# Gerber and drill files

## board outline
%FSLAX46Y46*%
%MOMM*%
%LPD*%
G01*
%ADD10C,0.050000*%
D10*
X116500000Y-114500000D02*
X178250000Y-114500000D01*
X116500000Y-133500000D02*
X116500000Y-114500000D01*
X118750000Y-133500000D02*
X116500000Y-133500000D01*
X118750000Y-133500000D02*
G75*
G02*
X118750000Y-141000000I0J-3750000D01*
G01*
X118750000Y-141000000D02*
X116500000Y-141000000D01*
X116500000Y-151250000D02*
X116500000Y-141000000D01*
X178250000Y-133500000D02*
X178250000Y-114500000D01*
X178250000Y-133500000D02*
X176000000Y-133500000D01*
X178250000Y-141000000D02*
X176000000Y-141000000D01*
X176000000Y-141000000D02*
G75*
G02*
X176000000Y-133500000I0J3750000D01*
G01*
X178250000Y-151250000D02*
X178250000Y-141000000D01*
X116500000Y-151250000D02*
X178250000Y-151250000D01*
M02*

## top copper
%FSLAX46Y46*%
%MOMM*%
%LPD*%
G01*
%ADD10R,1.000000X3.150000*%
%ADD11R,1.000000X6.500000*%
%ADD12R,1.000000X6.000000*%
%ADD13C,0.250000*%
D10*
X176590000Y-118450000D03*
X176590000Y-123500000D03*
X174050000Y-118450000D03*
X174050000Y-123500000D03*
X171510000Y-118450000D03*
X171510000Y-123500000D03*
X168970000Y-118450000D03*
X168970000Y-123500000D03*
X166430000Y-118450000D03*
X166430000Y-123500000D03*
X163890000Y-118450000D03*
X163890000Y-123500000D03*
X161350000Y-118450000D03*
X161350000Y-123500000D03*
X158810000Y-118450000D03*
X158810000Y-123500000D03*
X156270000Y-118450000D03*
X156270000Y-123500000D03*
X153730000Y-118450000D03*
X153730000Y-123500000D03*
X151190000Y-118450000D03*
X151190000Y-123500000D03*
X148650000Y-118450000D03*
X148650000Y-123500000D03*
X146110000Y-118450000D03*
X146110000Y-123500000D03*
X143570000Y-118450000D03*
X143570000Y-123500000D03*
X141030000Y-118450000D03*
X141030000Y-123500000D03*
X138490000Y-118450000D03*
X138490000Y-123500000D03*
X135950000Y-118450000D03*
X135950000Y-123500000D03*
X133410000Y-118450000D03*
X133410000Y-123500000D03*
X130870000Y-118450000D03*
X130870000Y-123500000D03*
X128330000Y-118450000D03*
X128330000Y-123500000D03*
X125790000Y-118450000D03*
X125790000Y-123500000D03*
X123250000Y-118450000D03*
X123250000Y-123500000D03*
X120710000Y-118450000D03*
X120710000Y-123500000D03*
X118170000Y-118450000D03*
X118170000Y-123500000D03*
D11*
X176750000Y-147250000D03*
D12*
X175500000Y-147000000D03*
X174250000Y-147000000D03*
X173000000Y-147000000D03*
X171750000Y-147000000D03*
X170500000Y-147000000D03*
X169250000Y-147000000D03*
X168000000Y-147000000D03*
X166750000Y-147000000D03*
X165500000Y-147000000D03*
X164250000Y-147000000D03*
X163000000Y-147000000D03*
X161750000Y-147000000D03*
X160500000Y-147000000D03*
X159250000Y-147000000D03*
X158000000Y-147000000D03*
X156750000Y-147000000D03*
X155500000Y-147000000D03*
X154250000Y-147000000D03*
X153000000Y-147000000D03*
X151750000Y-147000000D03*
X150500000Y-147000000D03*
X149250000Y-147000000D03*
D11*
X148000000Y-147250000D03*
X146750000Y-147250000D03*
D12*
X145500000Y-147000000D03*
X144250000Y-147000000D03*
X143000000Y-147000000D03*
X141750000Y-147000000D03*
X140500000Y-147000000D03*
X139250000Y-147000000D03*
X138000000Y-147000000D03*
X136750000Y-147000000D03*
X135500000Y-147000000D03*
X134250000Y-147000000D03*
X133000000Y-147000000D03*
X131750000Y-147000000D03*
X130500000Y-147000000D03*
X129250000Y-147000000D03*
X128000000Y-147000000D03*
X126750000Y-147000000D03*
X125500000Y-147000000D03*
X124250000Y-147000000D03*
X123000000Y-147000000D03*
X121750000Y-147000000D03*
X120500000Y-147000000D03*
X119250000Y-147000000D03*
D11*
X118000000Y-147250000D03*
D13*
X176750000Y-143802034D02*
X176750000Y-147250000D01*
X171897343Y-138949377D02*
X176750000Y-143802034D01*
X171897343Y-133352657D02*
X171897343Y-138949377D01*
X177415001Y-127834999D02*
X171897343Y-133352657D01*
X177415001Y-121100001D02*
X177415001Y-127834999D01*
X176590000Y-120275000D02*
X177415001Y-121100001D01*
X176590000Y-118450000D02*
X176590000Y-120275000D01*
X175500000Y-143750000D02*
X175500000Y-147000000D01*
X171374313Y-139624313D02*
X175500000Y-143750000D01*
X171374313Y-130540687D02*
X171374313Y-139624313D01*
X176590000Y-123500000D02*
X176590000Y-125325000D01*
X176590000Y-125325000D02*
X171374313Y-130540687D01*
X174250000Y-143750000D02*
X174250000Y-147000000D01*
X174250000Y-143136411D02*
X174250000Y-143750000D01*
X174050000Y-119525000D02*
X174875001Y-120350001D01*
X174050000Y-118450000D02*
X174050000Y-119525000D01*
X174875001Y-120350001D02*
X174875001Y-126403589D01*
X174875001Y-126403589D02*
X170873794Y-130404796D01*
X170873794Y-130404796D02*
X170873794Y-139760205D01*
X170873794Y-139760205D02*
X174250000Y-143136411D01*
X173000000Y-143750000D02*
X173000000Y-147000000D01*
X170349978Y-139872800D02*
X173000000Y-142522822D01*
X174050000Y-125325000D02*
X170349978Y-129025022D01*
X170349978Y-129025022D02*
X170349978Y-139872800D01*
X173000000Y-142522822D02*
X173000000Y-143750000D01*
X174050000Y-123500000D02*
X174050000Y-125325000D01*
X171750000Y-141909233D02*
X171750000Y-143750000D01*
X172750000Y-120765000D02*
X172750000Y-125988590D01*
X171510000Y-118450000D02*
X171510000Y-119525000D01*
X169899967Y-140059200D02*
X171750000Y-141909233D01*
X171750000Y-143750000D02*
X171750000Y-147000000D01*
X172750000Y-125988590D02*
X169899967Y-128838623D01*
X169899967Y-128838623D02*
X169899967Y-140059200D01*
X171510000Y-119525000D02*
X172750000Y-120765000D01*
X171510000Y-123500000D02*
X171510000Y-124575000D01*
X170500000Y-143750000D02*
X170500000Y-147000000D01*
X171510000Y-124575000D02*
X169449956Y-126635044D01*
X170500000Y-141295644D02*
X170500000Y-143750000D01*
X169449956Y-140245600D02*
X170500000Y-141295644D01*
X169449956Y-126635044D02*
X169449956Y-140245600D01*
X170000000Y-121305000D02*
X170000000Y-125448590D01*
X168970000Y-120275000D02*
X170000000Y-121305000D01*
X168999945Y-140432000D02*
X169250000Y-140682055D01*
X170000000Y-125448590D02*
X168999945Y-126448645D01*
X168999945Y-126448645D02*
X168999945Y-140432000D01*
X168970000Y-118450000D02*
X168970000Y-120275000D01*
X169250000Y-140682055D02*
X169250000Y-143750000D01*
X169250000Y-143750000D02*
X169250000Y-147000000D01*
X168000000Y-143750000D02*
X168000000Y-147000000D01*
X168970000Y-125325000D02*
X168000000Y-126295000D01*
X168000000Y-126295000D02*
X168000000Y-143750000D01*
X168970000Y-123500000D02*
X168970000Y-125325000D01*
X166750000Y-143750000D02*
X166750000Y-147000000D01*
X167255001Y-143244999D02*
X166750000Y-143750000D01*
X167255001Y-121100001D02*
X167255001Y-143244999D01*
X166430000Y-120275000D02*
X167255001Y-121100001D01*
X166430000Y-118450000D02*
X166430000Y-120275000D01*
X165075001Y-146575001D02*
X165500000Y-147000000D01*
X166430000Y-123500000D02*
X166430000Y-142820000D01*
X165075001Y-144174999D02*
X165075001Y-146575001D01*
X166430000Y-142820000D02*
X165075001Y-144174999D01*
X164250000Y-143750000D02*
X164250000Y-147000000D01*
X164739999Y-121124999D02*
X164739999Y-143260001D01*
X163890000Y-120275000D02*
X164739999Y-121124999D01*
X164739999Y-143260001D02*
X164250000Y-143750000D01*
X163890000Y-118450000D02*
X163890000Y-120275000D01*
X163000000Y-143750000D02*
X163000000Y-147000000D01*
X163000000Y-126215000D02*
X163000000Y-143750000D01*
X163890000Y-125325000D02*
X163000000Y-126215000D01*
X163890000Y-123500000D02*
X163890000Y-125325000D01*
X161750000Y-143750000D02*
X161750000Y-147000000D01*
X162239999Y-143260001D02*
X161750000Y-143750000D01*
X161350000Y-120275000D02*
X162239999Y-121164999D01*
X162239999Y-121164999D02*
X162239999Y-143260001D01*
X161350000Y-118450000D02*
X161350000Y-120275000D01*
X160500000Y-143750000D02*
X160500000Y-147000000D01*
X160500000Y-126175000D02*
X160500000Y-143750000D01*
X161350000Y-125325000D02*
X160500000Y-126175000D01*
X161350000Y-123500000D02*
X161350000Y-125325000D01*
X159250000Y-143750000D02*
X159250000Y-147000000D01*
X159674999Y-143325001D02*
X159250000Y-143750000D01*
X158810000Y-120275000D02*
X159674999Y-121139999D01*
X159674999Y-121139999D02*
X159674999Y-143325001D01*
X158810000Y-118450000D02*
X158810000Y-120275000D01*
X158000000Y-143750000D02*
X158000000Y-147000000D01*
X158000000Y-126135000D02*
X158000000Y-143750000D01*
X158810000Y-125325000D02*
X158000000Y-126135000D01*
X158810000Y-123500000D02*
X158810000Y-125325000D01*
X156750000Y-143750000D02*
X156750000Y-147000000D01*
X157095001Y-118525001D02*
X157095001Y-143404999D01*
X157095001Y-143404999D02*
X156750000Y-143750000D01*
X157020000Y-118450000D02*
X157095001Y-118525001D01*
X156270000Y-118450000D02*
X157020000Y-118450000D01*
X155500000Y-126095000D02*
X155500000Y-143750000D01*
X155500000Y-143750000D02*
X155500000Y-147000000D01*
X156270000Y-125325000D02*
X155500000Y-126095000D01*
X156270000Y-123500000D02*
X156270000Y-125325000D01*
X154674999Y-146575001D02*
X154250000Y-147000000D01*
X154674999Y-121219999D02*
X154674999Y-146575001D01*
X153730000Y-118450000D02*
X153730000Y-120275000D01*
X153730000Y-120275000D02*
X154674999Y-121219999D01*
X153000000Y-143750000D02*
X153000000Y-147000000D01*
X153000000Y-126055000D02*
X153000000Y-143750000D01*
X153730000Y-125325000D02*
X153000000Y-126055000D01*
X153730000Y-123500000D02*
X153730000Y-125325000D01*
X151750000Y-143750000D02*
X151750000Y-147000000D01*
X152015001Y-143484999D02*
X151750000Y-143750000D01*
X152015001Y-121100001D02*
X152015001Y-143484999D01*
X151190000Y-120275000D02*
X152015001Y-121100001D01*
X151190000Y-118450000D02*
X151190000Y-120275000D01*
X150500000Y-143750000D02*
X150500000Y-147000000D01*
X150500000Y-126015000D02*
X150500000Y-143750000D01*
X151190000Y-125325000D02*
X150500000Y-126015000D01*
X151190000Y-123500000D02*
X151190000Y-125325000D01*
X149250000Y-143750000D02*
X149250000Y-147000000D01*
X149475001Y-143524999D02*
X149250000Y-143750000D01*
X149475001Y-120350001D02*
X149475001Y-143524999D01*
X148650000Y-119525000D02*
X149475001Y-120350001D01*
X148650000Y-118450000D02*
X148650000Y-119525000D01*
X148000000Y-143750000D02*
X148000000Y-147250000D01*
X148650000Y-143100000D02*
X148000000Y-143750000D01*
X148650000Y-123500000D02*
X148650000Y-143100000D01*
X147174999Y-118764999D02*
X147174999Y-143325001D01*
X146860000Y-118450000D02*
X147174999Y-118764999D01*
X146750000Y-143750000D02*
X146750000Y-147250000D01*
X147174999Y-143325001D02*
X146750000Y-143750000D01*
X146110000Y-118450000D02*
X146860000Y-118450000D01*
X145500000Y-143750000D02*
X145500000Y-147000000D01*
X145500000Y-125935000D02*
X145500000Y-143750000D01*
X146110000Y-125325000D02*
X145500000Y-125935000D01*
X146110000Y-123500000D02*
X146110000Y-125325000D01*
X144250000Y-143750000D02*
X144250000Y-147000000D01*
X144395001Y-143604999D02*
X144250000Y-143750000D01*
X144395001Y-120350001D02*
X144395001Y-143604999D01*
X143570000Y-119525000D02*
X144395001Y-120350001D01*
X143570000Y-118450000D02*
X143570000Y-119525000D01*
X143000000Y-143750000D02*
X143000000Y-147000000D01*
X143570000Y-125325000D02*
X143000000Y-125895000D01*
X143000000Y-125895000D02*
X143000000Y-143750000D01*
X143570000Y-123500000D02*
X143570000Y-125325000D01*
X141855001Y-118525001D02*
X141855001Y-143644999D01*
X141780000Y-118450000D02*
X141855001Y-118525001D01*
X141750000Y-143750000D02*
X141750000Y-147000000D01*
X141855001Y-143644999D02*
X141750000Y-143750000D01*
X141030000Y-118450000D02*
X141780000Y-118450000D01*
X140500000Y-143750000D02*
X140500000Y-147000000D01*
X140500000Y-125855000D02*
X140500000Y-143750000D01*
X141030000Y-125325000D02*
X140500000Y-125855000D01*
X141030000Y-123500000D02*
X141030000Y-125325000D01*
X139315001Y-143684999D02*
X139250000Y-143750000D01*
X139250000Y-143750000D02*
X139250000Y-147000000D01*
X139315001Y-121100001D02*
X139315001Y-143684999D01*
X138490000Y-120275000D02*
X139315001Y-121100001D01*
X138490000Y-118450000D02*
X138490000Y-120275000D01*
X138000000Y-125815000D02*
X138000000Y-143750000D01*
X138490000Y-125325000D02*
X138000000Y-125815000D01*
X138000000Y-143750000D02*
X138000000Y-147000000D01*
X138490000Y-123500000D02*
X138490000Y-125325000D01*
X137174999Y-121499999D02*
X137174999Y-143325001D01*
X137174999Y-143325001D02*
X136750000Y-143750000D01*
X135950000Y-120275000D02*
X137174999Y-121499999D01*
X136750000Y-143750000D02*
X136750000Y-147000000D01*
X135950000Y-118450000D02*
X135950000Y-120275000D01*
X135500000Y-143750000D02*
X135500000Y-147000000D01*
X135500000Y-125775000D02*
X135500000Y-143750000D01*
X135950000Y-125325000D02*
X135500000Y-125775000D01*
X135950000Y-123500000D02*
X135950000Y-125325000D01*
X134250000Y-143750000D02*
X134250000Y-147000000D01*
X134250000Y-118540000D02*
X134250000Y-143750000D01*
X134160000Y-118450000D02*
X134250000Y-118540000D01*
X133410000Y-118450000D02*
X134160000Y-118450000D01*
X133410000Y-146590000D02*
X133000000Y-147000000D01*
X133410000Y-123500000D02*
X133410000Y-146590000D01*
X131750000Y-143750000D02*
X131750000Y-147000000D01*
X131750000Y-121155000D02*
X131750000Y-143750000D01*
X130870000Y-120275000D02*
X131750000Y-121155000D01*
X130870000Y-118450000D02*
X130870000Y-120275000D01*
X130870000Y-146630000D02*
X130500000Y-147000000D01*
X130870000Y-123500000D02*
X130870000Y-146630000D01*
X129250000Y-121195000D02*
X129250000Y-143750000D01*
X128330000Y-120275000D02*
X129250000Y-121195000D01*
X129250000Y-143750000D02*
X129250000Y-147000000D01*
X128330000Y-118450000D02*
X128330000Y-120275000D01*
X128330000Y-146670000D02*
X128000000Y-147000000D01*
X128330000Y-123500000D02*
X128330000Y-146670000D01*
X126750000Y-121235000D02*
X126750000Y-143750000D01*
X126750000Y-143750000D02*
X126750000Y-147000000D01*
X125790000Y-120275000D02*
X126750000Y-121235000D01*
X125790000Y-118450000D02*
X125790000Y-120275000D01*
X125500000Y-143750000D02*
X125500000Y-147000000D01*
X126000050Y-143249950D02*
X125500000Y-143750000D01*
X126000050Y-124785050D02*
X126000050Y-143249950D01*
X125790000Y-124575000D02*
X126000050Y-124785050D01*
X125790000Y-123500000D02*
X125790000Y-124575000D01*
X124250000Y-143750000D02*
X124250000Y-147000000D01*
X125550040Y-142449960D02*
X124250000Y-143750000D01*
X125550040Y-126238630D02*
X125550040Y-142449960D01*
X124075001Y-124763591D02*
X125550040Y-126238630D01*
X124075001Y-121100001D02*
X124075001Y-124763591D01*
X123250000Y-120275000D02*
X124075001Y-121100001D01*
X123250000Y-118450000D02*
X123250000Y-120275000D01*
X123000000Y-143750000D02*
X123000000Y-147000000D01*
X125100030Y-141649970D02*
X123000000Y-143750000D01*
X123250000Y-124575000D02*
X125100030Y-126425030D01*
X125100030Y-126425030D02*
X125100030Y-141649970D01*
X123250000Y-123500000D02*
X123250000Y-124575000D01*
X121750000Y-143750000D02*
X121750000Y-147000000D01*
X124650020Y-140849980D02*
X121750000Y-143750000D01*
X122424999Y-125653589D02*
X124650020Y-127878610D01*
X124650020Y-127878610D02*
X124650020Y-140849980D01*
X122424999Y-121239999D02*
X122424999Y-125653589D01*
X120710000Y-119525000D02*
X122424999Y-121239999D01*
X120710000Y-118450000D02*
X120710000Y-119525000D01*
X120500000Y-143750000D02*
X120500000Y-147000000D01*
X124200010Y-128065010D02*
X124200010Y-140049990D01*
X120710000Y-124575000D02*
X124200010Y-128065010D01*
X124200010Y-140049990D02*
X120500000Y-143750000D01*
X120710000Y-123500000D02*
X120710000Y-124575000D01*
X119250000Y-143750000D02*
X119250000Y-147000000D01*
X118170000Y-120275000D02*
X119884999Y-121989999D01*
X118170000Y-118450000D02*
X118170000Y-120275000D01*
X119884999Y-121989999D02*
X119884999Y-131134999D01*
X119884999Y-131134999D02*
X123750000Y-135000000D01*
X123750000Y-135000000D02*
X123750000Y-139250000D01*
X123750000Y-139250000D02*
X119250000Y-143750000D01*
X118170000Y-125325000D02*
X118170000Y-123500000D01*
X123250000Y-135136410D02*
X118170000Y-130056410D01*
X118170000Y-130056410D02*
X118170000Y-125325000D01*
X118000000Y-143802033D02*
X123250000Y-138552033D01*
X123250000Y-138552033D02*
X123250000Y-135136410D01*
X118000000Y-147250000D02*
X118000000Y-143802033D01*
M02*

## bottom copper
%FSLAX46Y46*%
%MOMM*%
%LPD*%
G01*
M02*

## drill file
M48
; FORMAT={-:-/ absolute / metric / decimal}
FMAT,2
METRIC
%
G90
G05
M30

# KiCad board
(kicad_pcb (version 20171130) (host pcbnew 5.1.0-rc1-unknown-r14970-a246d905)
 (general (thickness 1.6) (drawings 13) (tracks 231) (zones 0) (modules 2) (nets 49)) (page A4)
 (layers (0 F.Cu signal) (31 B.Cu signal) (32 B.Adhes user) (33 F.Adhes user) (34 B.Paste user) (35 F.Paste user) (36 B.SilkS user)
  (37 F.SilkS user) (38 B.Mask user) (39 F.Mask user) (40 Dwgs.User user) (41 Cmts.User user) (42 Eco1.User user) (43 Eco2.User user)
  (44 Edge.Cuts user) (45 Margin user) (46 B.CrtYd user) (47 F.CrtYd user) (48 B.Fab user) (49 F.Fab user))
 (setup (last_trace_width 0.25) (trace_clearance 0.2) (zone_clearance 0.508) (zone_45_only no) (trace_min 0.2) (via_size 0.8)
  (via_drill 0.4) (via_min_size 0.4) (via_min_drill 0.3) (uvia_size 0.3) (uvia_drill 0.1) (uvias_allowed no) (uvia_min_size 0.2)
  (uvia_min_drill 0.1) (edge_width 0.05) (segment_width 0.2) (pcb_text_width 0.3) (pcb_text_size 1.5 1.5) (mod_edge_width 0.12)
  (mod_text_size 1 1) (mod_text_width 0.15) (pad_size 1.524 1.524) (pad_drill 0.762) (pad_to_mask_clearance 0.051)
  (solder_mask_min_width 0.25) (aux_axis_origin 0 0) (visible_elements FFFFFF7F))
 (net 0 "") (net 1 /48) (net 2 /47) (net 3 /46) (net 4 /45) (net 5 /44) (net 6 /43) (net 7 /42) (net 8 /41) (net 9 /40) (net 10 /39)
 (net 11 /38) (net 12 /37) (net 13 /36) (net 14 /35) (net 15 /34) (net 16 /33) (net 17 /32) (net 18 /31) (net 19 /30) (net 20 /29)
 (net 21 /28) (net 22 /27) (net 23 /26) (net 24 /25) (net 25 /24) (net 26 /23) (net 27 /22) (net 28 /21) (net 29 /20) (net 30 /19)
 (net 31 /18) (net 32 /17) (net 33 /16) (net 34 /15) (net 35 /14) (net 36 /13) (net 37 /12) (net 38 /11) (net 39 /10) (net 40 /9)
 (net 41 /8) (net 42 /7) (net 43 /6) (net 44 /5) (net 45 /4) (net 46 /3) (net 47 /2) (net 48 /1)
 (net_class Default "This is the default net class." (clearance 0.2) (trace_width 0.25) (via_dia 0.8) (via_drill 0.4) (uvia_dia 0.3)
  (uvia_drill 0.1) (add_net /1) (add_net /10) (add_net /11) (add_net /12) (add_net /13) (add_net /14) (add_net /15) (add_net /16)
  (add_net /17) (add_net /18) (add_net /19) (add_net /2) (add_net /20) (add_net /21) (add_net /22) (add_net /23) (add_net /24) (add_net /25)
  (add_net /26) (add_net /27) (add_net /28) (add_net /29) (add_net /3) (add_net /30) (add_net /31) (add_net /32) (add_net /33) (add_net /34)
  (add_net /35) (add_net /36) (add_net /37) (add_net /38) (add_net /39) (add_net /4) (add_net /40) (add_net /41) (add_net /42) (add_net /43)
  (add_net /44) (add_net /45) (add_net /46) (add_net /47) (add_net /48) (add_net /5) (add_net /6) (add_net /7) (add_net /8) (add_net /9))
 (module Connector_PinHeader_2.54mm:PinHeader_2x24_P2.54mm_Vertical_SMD (layer F.Cu) (at 147.38 120.975 90)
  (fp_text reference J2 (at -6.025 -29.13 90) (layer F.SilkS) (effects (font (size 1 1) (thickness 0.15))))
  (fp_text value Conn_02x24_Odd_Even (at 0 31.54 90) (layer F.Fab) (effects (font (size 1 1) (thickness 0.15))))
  (pad 48 smd rect (at 2.525 29.21 90) (size 3.15 1) (layers F.Cu F.Paste F.Mask) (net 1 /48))
  (pad 47 smd rect (at -2.525 29.21 90) (size 3.15 1) (layers F.Cu F.Paste F.Mask) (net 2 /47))
  (pad 46 smd rect (at 2.525 26.67 90) (size 3.15 1) (layers F.Cu F.Paste F.Mask) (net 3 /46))
  (pad 45 smd rect (at -2.525 26.67 90) (size 3.15 1) (layers F.Cu F.Paste F.Mask) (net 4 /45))
  (pad 44 smd rect (at 2.525 24.13 90) (size 3.15 1) (layers F.Cu F.Paste F.Mask) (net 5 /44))
  (pad 43 smd rect (at -2.525 24.13 90) (size 3.15 1) (layers F.Cu F.Paste F.Mask) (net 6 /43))
  (pad 42 smd rect (at 2.525 21.59 90) (size 3.15 1) (layers F.Cu F.Paste F.Mask) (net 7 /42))
  (pad 41 smd rect (at -2.525 21.59 90) (size 3.15 1) (layers F.Cu F.Paste F.Mask) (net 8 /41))
  (pad 40 smd rect (at 2.525 19.05 90) (size 3.15 1) (layers F.Cu F.Paste F.Mask) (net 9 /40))
  (pad 39 smd rect (at -2.525 19.05 90) (size 3.15 1) (layers F.Cu F.Paste F.Mask) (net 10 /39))
  (pad 38 smd rect (at 2.525 16.51 90) (size 3.15 1) (layers F.Cu F.Paste F.Mask) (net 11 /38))
  (pad 37 smd rect (at -2.525 16.51 90) (size 3.15 1) (layers F.Cu F.Paste F.Mask) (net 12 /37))
  (pad 36 smd rect (at 2.525 13.97 90) (size 3.15 1) (layers F.Cu F.Paste F.Mask) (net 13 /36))
  (pad 35 smd rect (at -2.525 13.97 90) (size 3.15 1) (layers F.Cu F.Paste F.Mask) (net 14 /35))
  (pad 34 smd rect (at 2.525 11.43 90) (size 3.15 1) (layers F.Cu F.Paste F.Mask) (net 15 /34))
  (pad 33 smd rect (at -2.525 11.43 90) (size 3.15 1) (layers F.Cu F.Paste F.Mask) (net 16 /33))
  (pad 32 smd rect (at 2.525 8.89 90) (size 3.15 1) (layers F.Cu F.Paste F.Mask) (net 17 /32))
  (pad 31 smd rect (at -2.525 8.89 90) (size 3.15 1) (layers F.Cu F.Paste F.Mask) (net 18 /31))
  (pad 30 smd rect (at 2.525 6.35 90) (size 3.15 1) (layers F.Cu F.Paste F.Mask) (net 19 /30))
  (pad 29 smd rect (at -2.525 6.35 90) (size 3.15 1) (layers F.Cu F.Paste F.Mask) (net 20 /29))
  (pad 28 smd rect (at 2.525 3.81 90) (size 3.15 1) (layers F.Cu F.Paste F.Mask) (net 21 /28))
  (pad 27 smd rect (at -2.525 3.81 90) (size 3.15 1) (layers F.Cu F.Paste F.Mask) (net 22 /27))
  (pad 26 smd rect (at 2.525 1.27 90) (size 3.15 1) (layers F.Cu F.Paste F.Mask) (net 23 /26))
  (pad 25 smd rect (at -2.525 1.27 90) (size 3.15 1) (layers F.Cu F.Paste F.Mask) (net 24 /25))
  (pad 24 smd rect (at 2.525 -1.27 90) (size 3.15 1) (layers F.Cu F.Paste F.Mask) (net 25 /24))
  (pad 23 smd rect (at -2.525 -1.27 90) (size 3.15 1) (layers F.Cu F.Paste F.Mask) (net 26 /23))
  (pad 22 smd rect (at 2.525 -3.81 90) (size 3.15 1) (layers F.Cu F.Paste F.Mask) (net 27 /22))
  (pad 21 smd rect (at -2.525 -3.81 90) (size 3.15 1) (layers F.Cu F.Paste F.Mask) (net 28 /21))
  (pad 20 smd rect (at 2.525 -6.35 90) (size 3.15 1) (layers F.Cu F.Paste F.Mask) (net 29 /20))
  (pad 19 smd rect (at -2.525 -6.35 90) (size 3.15 1) (layers F.Cu F.Paste F.Mask) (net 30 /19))
  (pad 18 smd rect (at 2.525 -8.89 90) (size 3.15 1) (layers F.Cu F.Paste F.Mask) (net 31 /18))
  (pad 17 smd rect (at -2.525 -8.89 90) (size 3.15 1) (layers F.Cu F.Paste F.Mask) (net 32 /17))
  (pad 16 smd rect (at 2.525 -11.43 90) (size 3.15 1) (layers F.Cu F.Paste F.Mask) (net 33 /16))
  (pad 15 smd rect (at -2.525 -11.43 90) (size 3.15 1) (layers F.Cu F.Paste F.Mask) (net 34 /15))
  (pad 14 smd rect (at 2.525 -13.97 90) (size 3.15 1) (layers F.Cu F.Paste F.Mask) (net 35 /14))
  (pad 13 smd rect (at -2.525 -13.97 90) (size 3.15 1) (layers F.Cu F.Paste F.Mask) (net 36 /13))
  (pad 12 smd rect (at 2.525 -16.51 90) (size 3.15 1) (layers F.Cu F.Paste F.Mask) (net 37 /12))
  (pad 11 smd rect (at -2.525 -16.51 90) (size 3.15 1) (layers F.Cu F.Paste F.Mask) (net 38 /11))
  (pad 10 smd rect (at 2.525 -19.05 90) (size 3.15 1) (layers F.Cu F.Paste F.Mask) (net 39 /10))
  (pad 9 smd rect (at -2.525 -19.05 90) (size 3.15 1) (layers F.Cu F.Paste F.Mask) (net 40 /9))
  (pad 8 smd rect (at 2.525 -21.59 90) (size 3.15 1) (layers F.Cu F.Paste F.Mask) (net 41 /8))
  (pad 7 smd rect (at -2.525 -21.59 90) (size 3.15 1) (layers F.Cu F.Paste F.Mask) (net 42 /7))
  (pad 6 smd rect (at 2.525 -24.13 90) (size 3.15 1) (layers F.Cu F.Paste F.Mask) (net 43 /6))
  (pad 5 smd rect (at -2.525 -24.13 90) (size 3.15 1) (layers F.Cu F.Paste F.Mask) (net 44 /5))
  (pad 4 smd rect (at 2.525 -26.67 90) (size 3.15 1) (layers F.Cu F.Paste F.Mask) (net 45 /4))
  (pad 3 smd rect (at -2.525 -26.67 90) (size 3.15 1) (layers F.Cu F.Paste F.Mask) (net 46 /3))
  (pad 2 smd rect (at 2.525 -29.21 90) (size 3.15 1) (layers F.Cu F.Paste F.Mask) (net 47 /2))
  (pad 1 smd rect (at -2.525 -29.21 90) (size 3.15 1) (layers F.Cu F.Paste F.Mask) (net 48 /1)))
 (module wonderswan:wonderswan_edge (layer F.Cu) (at 147.375 147)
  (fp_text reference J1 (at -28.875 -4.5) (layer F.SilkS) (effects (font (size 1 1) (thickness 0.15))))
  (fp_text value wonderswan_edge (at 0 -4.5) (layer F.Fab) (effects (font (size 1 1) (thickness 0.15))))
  (pad 48 smd rect (at 29.375 0.25) (size 1 6.5) (layers F.Cu F.Paste F.Mask) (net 1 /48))
  (pad 47 smd rect (at 28.125 0) (size 1 6) (layers F.Cu F.Paste F.Mask) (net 2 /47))
  (pad 46 smd rect (at 26.875 0) (size 1 6) (layers F.Cu F.Paste F.Mask) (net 3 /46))
  (pad 45 smd rect (at 25.625 0) (size 1 6) (layers F.Cu F.Paste F.Mask) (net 4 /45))
  (pad 44 smd rect (at 24.375 0) (size 1 6) (layers F.Cu F.Paste F.Mask) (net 5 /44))
  (pad 43 smd rect (at 23.125 0) (size 1 6) (layers F.Cu F.Paste F.Mask) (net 6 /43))
  (pad 42 smd rect (at 21.875 0) (size 1 6) (layers F.Cu F.Paste F.Mask) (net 7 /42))
  (pad 41 smd rect (at 20.625 0) (size 1 6) (layers F.Cu F.Paste F.Mask) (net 8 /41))
  (pad 40 smd rect (at 19.375 0) (size 1 6) (layers F.Cu F.Paste F.Mask) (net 9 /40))
  (pad 39 smd rect (at 18.125 0) (size 1 6) (layers F.Cu F.Paste F.Mask) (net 10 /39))
  (pad 38 smd rect (at 16.875 0) (size 1 6) (layers F.Cu F.Paste F.Mask) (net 11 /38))
  (pad 37 smd rect (at 15.625 0) (size 1 6) (layers F.Cu F.Paste F.Mask) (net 12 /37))
  (pad 36 smd rect (at 14.375 0) (size 1 6) (layers F.Cu F.Paste F.Mask) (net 13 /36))
  (pad 35 smd rect (at 13.125 0) (size 1 6) (layers F.Cu F.Paste F.Mask) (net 14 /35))
  (pad 34 smd rect (at 11.875 0) (size 1 6) (layers F.Cu F.Paste F.Mask) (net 15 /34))
  (pad 33 smd rect (at 10.625 0) (size 1 6) (layers F.Cu F.Paste F.Mask) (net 16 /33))
  (pad 32 smd rect (at 9.375 0) (size 1 6) (layers F.Cu F.Paste F.Mask) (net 17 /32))
  (pad 31 smd rect (at 8.125 0) (size 1 6) (layers F.Cu F.Paste F.Mask) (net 18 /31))
  (pad 30 smd rect (at 6.875 0) (size 1 6) (layers F.Cu F.Paste F.Mask) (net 19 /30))
  (pad 29 smd rect (at 5.625 0) (size 1 6) (layers F.Cu F.Paste F.Mask) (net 20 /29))
  (pad 28 smd rect (at 4.375 0) (size 1 6) (layers F.Cu F.Paste F.Mask) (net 21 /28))
  (pad 27 smd rect (at 3.125 0) (size 1 6) (layers F.Cu F.Paste F.Mask) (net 22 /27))
  (pad 26 smd rect (at 1.875 0) (size 1 6) (layers F.Cu F.Paste F.Mask) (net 23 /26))
  (pad 25 smd rect (at 0.625 0.25) (size 1 6.5) (layers F.Cu F.Paste F.Mask) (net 24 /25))
  (pad 24 smd rect (at -0.625 0.25) (size 1 6.5) (layers F.Cu F.Paste F.Mask) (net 25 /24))
  (pad 23 smd rect (at -1.875 0) (size 1 6) (layers F.Cu F.Paste F.Mask) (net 26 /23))
  (pad 22 smd rect (at -3.125 0) (size 1 6) (layers F.Cu F.Paste F.Mask) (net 27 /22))
  (pad 21 smd rect (at -4.375 0) (size 1 6) (layers F.Cu F.Paste F.Mask) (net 28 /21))
  (pad 20 smd rect (at -5.625 0) (size 1 6) (layers F.Cu F.Paste F.Mask) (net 29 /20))
  (pad 19 smd rect (at -6.875 0) (size 1 6) (layers F.Cu F.Paste F.Mask) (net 30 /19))
  (pad 18 smd rect (at -8.125 0) (size 1 6) (layers F.Cu F.Paste F.Mask) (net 31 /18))
  (pad 17 smd rect (at -9.375 0) (size 1 6) (layers F.Cu F.Paste F.Mask) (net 32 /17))
  (pad 16 smd rect (at -10.625 0) (size 1 6) (layers F.Cu F.Paste F.Mask) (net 33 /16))
  (pad 15 smd rect (at -11.875 0) (size 1 6) (layers F.Cu F.Paste F.Mask) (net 34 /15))
  (pad 14 smd rect (at -13.125 0) (size 1 6) (layers F.Cu F.Paste F.Mask) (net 35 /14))
  (pad 13 smd rect (at -14.375 0) (size 1 6) (layers F.Cu F.Paste F.Mask) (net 36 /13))
  (pad 12 smd rect (at -15.625 0) (size 1 6) (layers F.Cu F.Paste F.Mask) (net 37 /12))
  (pad 11 smd rect (at -16.875 0) (size 1 6) (layers F.Cu F.Paste F.Mask) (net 38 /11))
  (pad 10 smd rect (at -18.125 0) (size 1 6) (layers F.Cu F.Paste F.Mask) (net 39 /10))
  (pad 9 smd rect (at -19.375 0) (size 1 6) (layers F.Cu F.Paste F.Mask) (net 40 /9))
  (pad 8 smd rect (at -20.625 0) (size 1 6) (layers F.Cu F.Paste F.Mask) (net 41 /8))
  (pad 7 smd rect (at -21.875 0) (size 1 6) (layers F.Cu F.Paste F.Mask) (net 42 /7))
  (pad 6 smd rect (at -23.125 0) (size 1 6) (layers F.Cu F.Paste F.Mask) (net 43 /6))
  (pad 5 smd rect (at -24.375 0) (size 1 6) (layers F.Cu F.Paste F.Mask) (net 44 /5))
  (pad 4 smd rect (at -25.625 0) (size 1 6) (layers F.Cu F.Paste F.Mask) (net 45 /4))
  (pad 3 smd rect (at -26.875 0) (size 1 6) (layers F.Cu F.Paste F.Mask) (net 46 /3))
  (pad 2 smd rect (at -28.125 0) (size 1 6) (layers F.Cu F.Paste F.Mask) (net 47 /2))
  (pad 1 smd rect (at -29.375 0.25) (size 1 6.5) (layers F.Cu F.Paste F.Mask) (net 48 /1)))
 (gr_line (start 116.5 114.5) (end 178.25 114.5) (layer Edge.Cuts) (width 0.05))
 (gr_line (start 116.5 133.5) (end 116.5 114.5) (layer Edge.Cuts) (width 0.05))
 (gr_line (start 118.75 133.5) (end 116.5 133.5) (layer Edge.Cuts) (width 0.05))
 (gr_arc (start 118.75 137.25) (end 118.75 141) (angle -180) (layer Edge.Cuts) (width 0.05))
 (gr_line (start 118.75 141) (end 116.5 141) (layer Edge.Cuts) (width 0.05))
 (gr_line (start 116.5 151.25) (end 116.5 141) (layer Edge.Cuts) (width 0.05))
 (gr_line (start 178.25 133.5) (end 178.25 114.5) (layer Edge.Cuts) (width 0.05))
 (gr_line (start 178.25 133.5) (end 176 133.5) (layer Edge.Cuts) (width 0.05))
 (gr_line (start 178.25 141) (end 176 141) (layer Edge.Cuts) (width 0.05))
 (gr_arc (start 176 137.25) (end 176 133.5) (angle -180) (layer Edge.Cuts) (width 0.05))
 (gr_line (start 178.25 151.25) (end 178.25 141) (layer Edge.Cuts) (width 0.05))
 (gr_line (start 116.5 151.25) (end 178.25 151.25) (layer Edge.Cuts) (width 0.05))
 (segment (start 176.75 143.802034) (end 176.75 147.25) (width 0.25) (layer F.Cu) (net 1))
 (segment (start 171.897343 138.949377) (end 176.75 143.802034) (width 0.25) (layer F.Cu) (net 1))
 (segment (start 171.897343 133.352657) (end 171.897343 138.949377) (width 0.25) (layer F.Cu) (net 1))
 (segment (start 177.415001 127.834999) (end 171.897343 133.352657) (width 0.25) (layer F.Cu) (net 1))
 (segment (start 177.415001 121.100001) (end 177.415001 127.834999) (width 0.25) (layer F.Cu) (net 1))
 (segment (start 176.59 120.275) (end 177.415001 121.100001) (width 0.25) (layer F.Cu) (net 1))
 (segment (start 176.59 118.45) (end 176.59 120.275) (width 0.25) (layer F.Cu) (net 1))
 (segment (start 175.5 143.75) (end 175.5 147) (width 0.25) (layer F.Cu) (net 2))
 (segment (start 171.374313 139.624313) (end 175.5 143.75) (width 0.25) (layer F.Cu) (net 2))
 (segment (start 171.374313 130.540687) (end 171.374313 139.624313) (width 0.25) (layer F.Cu) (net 2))
 (segment (start 176.59 123.5) (end 176.59 125.325) (width 0.25) (layer F.Cu) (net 2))
 (segment (start 176.59 125.325) (end 171.374313 130.540687) (width 0.25) (layer F.Cu) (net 2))
 (segment (start 174.25 143.75) (end 174.25 147) (width 0.25) (layer F.Cu) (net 3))
 (segment (start 174.25 143.136411) (end 174.25 143.75) (width 0.25) (layer F.Cu) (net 3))
 (segment (start 174.05 119.525) (end 174.875001 120.350001) (width 0.25) (layer F.Cu) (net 3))
 (segment (start 174.05 118.45) (end 174.05 119.525) (width 0.25) (layer F.Cu) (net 3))
 (segment (start 174.875001 120.350001) (end 174.875001 126.403589) (width 0.25) (layer F.Cu) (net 3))
 (segment (start 174.875001 126.403589) (end 170.873794 130.404796) (width 0.25) (layer F.Cu) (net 3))
 (segment (start 170.873794 130.404796) (end 170.873794 139.760205) (width 0.25) (layer F.Cu) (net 3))
 (segment (start 170.873794 139.760205) (end 174.25 143.136411) (width 0.25) (layer F.Cu) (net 3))
 (segment (start 173 143.75) (end 173 147) (width 0.25) (layer F.Cu) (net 4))
 (segment (start 170.349978 139.8728) (end 173 142.522822) (width 0.25) (layer F.Cu) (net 4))
 (segment (start 174.05 125.325) (end 170.349978 129.025022) (width 0.25) (layer F.Cu) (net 4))
 (segment (start 170.349978 129.025022) (end 170.349978 139.8728) (width 0.25) (layer F.Cu) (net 4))
 (segment (start 173 142.522822) (end 173 143.75) (width 0.25) (layer F.Cu) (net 4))
 (segment (start 174.05 123.5) (end 174.05 125.325) (width 0.25) (layer F.Cu) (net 4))
 (segment (start 171.75 141.909233) (end 171.75 143.75) (width 0.25) (layer F.Cu) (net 5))
 (segment (start 172.75 120.765) (end 172.75 125.98859) (width 0.25) (layer F.Cu) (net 5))
 (segment (start 171.51 118.45) (end 171.51 119.525) (width 0.25) (layer F.Cu) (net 5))
 (segment (start 169.899967 140.0592) (end 171.75 141.909233) (width 0.25) (layer F.Cu) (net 5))
 (segment (start 171.75 143.75) (end 171.75 147) (width 0.25) (layer F.Cu) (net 5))
 (segment (start 172.75 125.98859) (end 169.899967 128.838623) (width 0.25) (layer F.Cu) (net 5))
 (segment (start 169.899967 128.838623) (end 169.899967 140.0592) (width 0.25) (layer F.Cu) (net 5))
 (segment (start 171.51 119.525) (end 172.75 120.765) (width 0.25) (layer F.Cu) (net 5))
 (segment (start 171.51 123.5) (end 171.51 124.575) (width 0.25) (layer F.Cu) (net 6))
 (segment (start 170.5 143.75) (end 170.5 147) (width 0.25) (layer F.Cu) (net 6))
 (segment (start 171.51 124.575) (end 169.449956 126.635044) (width 0.25) (layer F.Cu) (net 6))
 (segment (start 170.5 141.295644) (end 170.5 143.75) (width 0.25) (layer F.Cu) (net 6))
 (segment (start 169.449956 140.2456) (end 170.5 141.295644) (width 0.25) (layer F.Cu) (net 6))
 (segment (start 169.449956 126.635044) (end 169.449956 140.2456) (width 0.25) (layer F.Cu) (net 6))
 (segment (start 170 121.305) (end 170 125.44859) (width 0.25) (layer F.Cu) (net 7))
 (segment (start 168.97 120.275) (end 170 121.305) (width 0.25) (layer F.Cu) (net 7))
 (segment (start 168.999945 140.432) (end 169.25 140.682055) (width 0.25) (layer F.Cu) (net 7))
 (segment (start 170 125.44859) (end 168.999945 126.448645) (width 0.25) (layer F.Cu) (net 7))
 (segment (start 168.999945 126.448645) (end 168.999945 140.432) (width 0.25) (layer F.Cu) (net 7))
 (segment (start 168.97 118.45) (end 168.97 120.275) (width 0.25) (layer F.Cu) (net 7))
 (segment (start 169.25 140.682055) (end 169.25 143.75) (width 0.25) (layer F.Cu) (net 7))
 (segment (start 169.25 143.75) (end 169.25 147) (width 0.25) (layer F.Cu) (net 7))
 (segment (start 168 143.75) (end 168 147) (width 0.25) (layer F.Cu) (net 8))
 (segment (start 168.97 125.325) (end 168 126.295) (width 0.25) (layer F.Cu) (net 8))
 (segment (start 168 126.295) (end 168 143.75) (width 0.25) (layer F.Cu) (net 8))
 (segment (start 168.97 123.5) (end 168.97 125.325) (width 0.25) (layer F.Cu) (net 8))
 (segment (start 166.75 143.75) (end 166.75 147) (width 0.25) (layer F.Cu) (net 9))
 (segment (start 167.255001 143.244999) (end 166.75 143.75) (width 0.25) (layer F.Cu) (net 9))
 (segment (start 167.255001 121.100001) (end 167.255001 143.244999) (width 0.25) (layer F.Cu) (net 9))
 (segment (start 166.43 120.275) (end 167.255001 121.100001) (width 0.25) (layer F.Cu) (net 9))
 (segment (start 166.43 118.45) (end 166.43 120.275) (width 0.25) (layer F.Cu) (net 9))
 (segment (start 165.075001 146.575001) (end 165.5 147) (width 0.25) (layer F.Cu) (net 10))
 (segment (start 166.43 123.5) (end 166.43 142.82) (width 0.25) (layer F.Cu) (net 10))
 (segment (start 165.075001 144.174999) (end 165.075001 146.575001) (width 0.25) (layer F.Cu) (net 10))
 (segment (start 166.43 142.82) (end 165.075001 144.174999) (width 0.25) (layer F.Cu) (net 10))
 (segment (start 164.25 143.75) (end 164.25 147) (width 0.25) (layer F.Cu) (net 11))
 (segment (start 164.739999 121.124999) (end 164.739999 143.260001) (width 0.25) (layer F.Cu) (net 11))
 (segment (start 163.89 120.275) (end 164.739999 121.124999) (width 0.25) (layer F.Cu) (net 11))
 (segment (start 164.739999 143.260001) (end 164.25 143.75) (width 0.25) (layer F.Cu) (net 11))
 (segment (start 163.89 118.45) (end 163.89 120.275) (width 0.25) (layer F.Cu) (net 11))
 (segment (start 163 143.75) (end 163 147) (width 0.25) (layer F.Cu) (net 12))
 (segment (start 163 126.215) (end 163 143.75) (width 0.25) (layer F.Cu) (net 12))
 (segment (start 163.89 125.325) (end 163 126.215) (width 0.25) (layer F.Cu) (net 12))
 (segment (start 163.89 123.5) (end 163.89 125.325) (width 0.25) (layer F.Cu) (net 12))
 (segment (start 161.75 143.75) (end 161.75 147) (width 0.25) (layer F.Cu) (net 13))
 (segment (start 162.239999 143.260001) (end 161.75 143.75) (width 0.25) (layer F.Cu) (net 13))
 (segment (start 161.35 120.275) (end 162.239999 121.164999) (width 0.25) (layer F.Cu) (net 13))
 (segment (start 162.239999 121.164999) (end 162.239999 143.260001) (width 0.25) (layer F.Cu) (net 13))
 (segment (start 161.35 118.45) (end 161.35 120.275) (width 0.25) (layer F.Cu) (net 13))
 (segment (start 160.5 143.75) (end 160.5 147) (width 0.25) (layer F.Cu) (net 14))
 (segment (start 160.5 126.175) (end 160.5 143.75) (width 0.25) (layer F.Cu) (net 14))
 (segment (start 161.35 125.325) (end 160.5 126.175) (width 0.25) (layer F.Cu) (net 14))
 (segment (start 161.35 123.5) (end 161.35 125.325) (width 0.25) (layer F.Cu) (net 14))
 (segment (start 159.25 143.75) (end 159.25 147) (width 0.25) (layer F.Cu) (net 15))
 (segment (start 159.674999 143.325001) (end 159.25 143.75) (width 0.25) (layer F.Cu) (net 15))
 (segment (start 158.81 120.275) (end 159.674999 121.139999) (width 0.25) (layer F.Cu) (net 15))
 (segment (start 159.674999 121.139999) (end 159.674999 143.325001) (width 0.25) (layer F.Cu) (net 15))
 (segment (start 158.81 118.45) (end 158.81 120.275) (width 0.25) (layer F.Cu) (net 15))
 (segment (start 158 143.75) (end 158 147) (width 0.25) (layer F.Cu) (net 16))
 (segment (start 158 126.135) (end 158 143.75) (width 0.25) (layer F.Cu) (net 16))
 (segment (start 158.81 125.325) (end 158 126.135) (width 0.25) (layer F.Cu) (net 16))
 (segment (start 158.81 123.5) (end 158.81 125.325) (width 0.25) (layer F.Cu) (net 16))
 (segment (start 156.75 143.75) (end 156.75 147) (width 0.25) (layer F.Cu) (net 17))
 (segment (start 157.095001 118.525001) (end 157.095001 143.404999) (width 0.25) (layer F.Cu) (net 17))
 (segment (start 157.095001 143.404999) (end 156.75 143.75) (width 0.25) (layer F.Cu) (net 17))
 (segment (start 157.02 118.45) (end 157.095001 118.525001) (width 0.25) (layer F.Cu) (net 17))
 (segment (start 156.27 118.45) (end 157.02 118.45) (width 0.25) (layer F.Cu) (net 17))
 (segment (start 155.5 126.095) (end 155.5 143.75) (width 0.25) (layer F.Cu) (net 18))
 (segment (start 155.5 143.75) (end 155.5 147) (width 0.25) (layer F.Cu) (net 18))
 (segment (start 156.27 125.325) (end 155.5 126.095) (width 0.25) (layer F.Cu) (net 18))
 (segment (start 156.27 123.5) (end 156.27 125.325) (width 0.25) (layer F.Cu) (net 18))
 (segment (start 154.674999 146.575001) (end 154.25 147) (width 0.25) (layer F.Cu) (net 19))
 (segment (start 154.674999 121.219999) (end 154.674999 146.575001) (width 0.25) (layer F.Cu) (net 19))
 (segment (start 153.73 118.45) (end 153.73 120.275) (width 0.25) (layer F.Cu) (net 19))
 (segment (start 153.73 120.275) (end 154.674999 121.219999) (width 0.25) (layer F.Cu) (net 19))
 (segment (start 153 143.75) (end 153 147) (width 0.25) (layer F.Cu) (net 20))
 (segment (start 153 126.055) (end 153 143.75) (width 0.25) (layer F.Cu) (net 20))
 (segment (start 153.73 125.325) (end 153 126.055) (width 0.25) (layer F.Cu) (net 20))
 (segment (start 153.73 123.5) (end 153.73 125.325) (width 0.25) (layer F.Cu) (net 20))
 (segment (start 151.75 143.75) (end 151.75 147) (width 0.25) (layer F.Cu) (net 21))
 (segment (start 152.015001 143.484999) (end 151.75 143.75) (width 0.25) (layer F.Cu) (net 21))
 (segment (start 152.015001 121.100001) (end 152.015001 143.484999) (width 0.25) (layer F.Cu) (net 21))
 (segment (start 151.19 120.275) (end 152.015001 121.100001) (width 0.25) (layer F.Cu) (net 21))
 (segment (start 151.19 118.45) (end 151.19 120.275) (width 0.25) (layer F.Cu) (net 21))
 (segment (start 150.5 143.75) (end 150.5 147) (width 0.25) (layer F.Cu) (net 22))
 (segment (start 150.5 126.015) (end 150.5 143.75) (width 0.25) (layer F.Cu) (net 22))
 (segment (start 151.19 125.325) (end 150.5 126.015) (width 0.25) (layer F.Cu) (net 22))
 (segment (start 151.19 123.5) (end 151.19 125.325) (width 0.25) (layer F.Cu) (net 22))
 (segment (start 149.25 143.75) (end 149.25 147) (width 0.25) (layer F.Cu) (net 23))
 (segment (start 149.475001 143.524999) (end 149.25 143.75) (width 0.25) (layer F.Cu) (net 23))
 (segment (start 149.475001 120.350001) (end 149.475001 143.524999) (width 0.25) (layer F.Cu) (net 23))
 (segment (start 148.65 119.525) (end 149.475001 120.350001) (width 0.25) (layer F.Cu) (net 23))
 (segment (start 148.65 118.45) (end 148.65 119.525) (width 0.25) (layer F.Cu) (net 23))
 (segment (start 148 143.75) (end 148 147.25) (width 0.25) (layer F.Cu) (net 24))
 (segment (start 148.65 143.1) (end 148 143.75) (width 0.25) (layer F.Cu) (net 24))
 (segment (start 148.65 123.5) (end 148.65 143.1) (width 0.25) (layer F.Cu) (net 24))
 (segment (start 147.174999 118.764999) (end 147.174999 143.325001) (width 0.25) (layer F.Cu) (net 25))
 (segment (start 146.86 118.45) (end 147.174999 118.764999) (width 0.25) (layer F.Cu) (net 25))
 (segment (start 146.75 143.75) (end 146.75 147.25) (width 0.25) (layer F.Cu) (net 25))
 (segment (start 147.174999 143.325001) (end 146.75 143.75) (width 0.25) (layer F.Cu) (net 25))
 (segment (start 146.11 118.45) (end 146.86 118.45) (width 0.25) (layer F.Cu) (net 25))
 (segment (start 145.5 143.75) (end 145.5 147) (width 0.25) (layer F.Cu) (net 26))
 (segment (start 145.5 125.935) (end 145.5 143.75) (width 0.25) (layer F.Cu) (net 26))
 (segment (start 146.11 125.325) (end 145.5 125.935) (width 0.25) (layer F.Cu) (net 26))
 (segment (start 146.11 123.5) (end 146.11 125.325) (width 0.25) (layer F.Cu) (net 26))
 (segment (start 144.25 143.75) (end 144.25 147) (width 0.25) (layer F.Cu) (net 27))
 (segment (start 144.395001 143.604999) (end 144.25 143.75) (width 0.25) (layer F.Cu) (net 27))
 (segment (start 144.395001 120.350001) (end 144.395001 143.604999) (width 0.25) (layer F.Cu) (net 27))
 (segment (start 143.57 119.525) (end 144.395001 120.350001) (width 0.25) (layer F.Cu) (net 27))
 (segment (start 143.57 118.45) (end 143.57 119.525) (width 0.25) (layer F.Cu) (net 27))
 (segment (start 143 143.75) (end 143 147) (width 0.25) (layer F.Cu) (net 28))
 (segment (start 143.57 125.325) (end 143 125.895) (width 0.25) (layer F.Cu) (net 28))
 (segment (start 143 125.895) (end 143 143.75) (width 0.25) (layer F.Cu) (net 28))
 (segment (start 143.57 123.5) (end 143.57 125.325) (width 0.25) (layer F.Cu) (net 28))
 (segment (start 141.855001 118.525001) (end 141.855001 143.644999) (width 0.25) (layer F.Cu) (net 29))
 (segment (start 141.78 118.45) (end 141.855001 118.525001) (width 0.25) (layer F.Cu) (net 29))
 (segment (start 141.75 143.75) (end 141.75 147) (width 0.25) (layer F.Cu) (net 29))
 (segment (start 141.855001 143.644999) (end 141.75 143.75) (width 0.25) (layer F.Cu) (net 29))
 (segment (start 141.03 118.45) (end 141.78 118.45) (width 0.25) (layer F.Cu) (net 29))
 (segment (start 140.5 143.75) (end 140.5 147) (width 0.25) (layer F.Cu) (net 30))
 (segment (start 140.5 125.855) (end 140.5 143.75) (width 0.25) (layer F.Cu) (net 30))
 (segment (start 141.03 125.325) (end 140.5 125.855) (width 0.25) (layer F.Cu) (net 30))
 (segment (start 141.03 123.5) (end 141.03 125.325) (width 0.25) (layer F.Cu) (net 30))
 (segment (start 139.315001 143.684999) (end 139.25 143.75) (width 0.25) (layer F.Cu) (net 31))
 (segment (start 139.25 143.75) (end 139.25 147) (width 0.25) (layer F.Cu) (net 31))
 (segment (start 139.315001 121.100001) (end 139.315001 143.684999) (width 0.25) (layer F.Cu) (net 31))
 (segment (start 138.49 120.275) (end 139.315001 121.100001) (width 0.25) (layer F.Cu) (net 31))
 (segment (start 138.49 118.45) (end 138.49 120.275) (width 0.25) (layer F.Cu) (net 31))
 (segment (start 138 125.815) (end 138 143.75) (width 0.25) (layer F.Cu) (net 32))
 (segment (start 138.49 125.325) (end 138 125.815) (width 0.25) (layer F.Cu) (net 32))
 (segment (start 138 143.75) (end 138 147) (width 0.25) (layer F.Cu) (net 32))
 (segment (start 138.49 123.5) (end 138.49 125.325) (width 0.25) (layer F.Cu) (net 32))
 (segment (start 137.174999 121.499999) (end 137.174999 143.325001) (width 0.25) (layer F.Cu) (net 33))
 (segment (start 137.174999 143.325001) (end 136.75 143.75) (width 0.25) (layer F.Cu) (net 33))
 (segment (start 135.95 120.275) (end 137.174999 121.499999) (width 0.25) (layer F.Cu) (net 33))
 (segment (start 136.75 143.75) (end 136.75 147) (width 0.25) (layer F.Cu) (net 33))
 (segment (start 135.95 118.45) (end 135.95 120.275) (width 0.25) (layer F.Cu) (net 33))
 (segment (start 135.5 143.75) (end 135.5 147) (width 0.25) (layer F.Cu) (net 34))
 (segment (start 135.5 125.775) (end 135.5 143.75) (width 0.25) (layer F.Cu) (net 34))
 (segment (start 135.95 125.325) (end 135.5 125.775) (width 0.25) (layer F.Cu) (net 34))
 (segment (start 135.95 123.5) (end 135.95 125.325) (width 0.25) (layer F.Cu) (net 34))
 (segment (start 134.25 143.75) (end 134.25 147) (width 0.25) (layer F.Cu) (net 35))
 (segment (start 134.25 118.54) (end 134.25 143.75) (width 0.25) (layer F.Cu) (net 35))
 (segment (start 134.16 118.45) (end 134.25 118.54) (width 0.25) (layer F.Cu) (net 35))
 (segment (start 133.41 118.45) (end 134.16 118.45) (width 0.25) (layer F.Cu) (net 35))
 (segment (start 133.41 146.59) (end 133 147) (width 0.25) (layer F.Cu) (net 36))
 (segment (start 133.41 123.5) (end 133.41 146.59) (width 0.25) (layer F.Cu) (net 36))
 (segment (start 131.75 143.75) (end 131.75 147) (width 0.25) (layer F.Cu) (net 37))
 (segment (start 131.75 121.155) (end 131.75 143.75) (width 0.25) (layer F.Cu) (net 37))
 (segment (start 130.87 120.275) (end 131.75 121.155) (width 0.25) (layer F.Cu) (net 37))
 (segment (start 130.87 118.45) (end 130.87 120.275) (width 0.25) (layer F.Cu) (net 37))
 (segment (start 130.87 146.63) (end 130.5 147) (width 0.25) (layer F.Cu) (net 38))
 (segment (start 130.87 123.5) (end 130.87 146.63) (width 0.25) (layer F.Cu) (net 38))
 (segment (start 129.25 121.195) (end 129.25 143.75) (width 0.25) (layer F.Cu) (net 39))
 (segment (start 128.33 120.275) (end 129.25 121.195) (width 0.25) (layer F.Cu) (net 39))
 (segment (start 129.25 143.75) (end 129.25 147) (width 0.25) (layer F.Cu) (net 39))
 (segment (start 128.33 118.45) (end 128.33 120.275) (width 0.25) (layer F.Cu) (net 39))
 (segment (start 128.33 146.67) (end 128 147) (width 0.25) (layer F.Cu) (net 40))
 (segment (start 128.33 123.5) (end 128.33 146.67) (width 0.25) (layer F.Cu) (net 40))
 (segment (start 126.75 121.235) (end 126.75 143.75) (width 0.25) (layer F.Cu) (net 41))
 (segment (start 126.75 143.75) (end 126.75 147) (width 0.25) (layer F.Cu) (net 41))
 (segment (start 125.79 120.275) (end 126.75 121.235) (width 0.25) (layer F.Cu) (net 41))
 (segment (start 125.79 118.45) (end 125.79 120.275) (width 0.25) (layer F.Cu) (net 41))
 (segment (start 125.5 143.75) (end 125.5 147) (width 0.25) (layer F.Cu) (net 42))
 (segment (start 126.00005 143.24995) (end 125.5 143.75) (width 0.25) (layer F.Cu) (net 42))
 (segment (start 126.00005 124.78505) (end 126.00005 143.24995) (width 0.25) (layer F.Cu) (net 42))
 (segment (start 125.79 124.575) (end 126.00005 124.78505) (width 0.25) (layer F.Cu) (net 42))
 (segment (start 125.79 123.5) (end 125.79 124.575) (width 0.25) (layer F.Cu) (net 42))
 (segment (start 124.25 143.75) (end 124.25 147) (width 0.25) (layer F.Cu) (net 43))
 (segment (start 125.55004 142.44996) (end 124.25 143.75) (width 0.25) (layer F.Cu) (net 43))
 (segment (start 125.55004 126.23863) (end 125.55004 142.44996) (width 0.25) (layer F.Cu) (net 43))
 (segment (start 124.075001 124.763591) (end 125.55004 126.23863) (width 0.25) (layer F.Cu) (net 43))
 (segment (start 124.075001 121.100001) (end 124.075001 124.763591) (width 0.25) (layer F.Cu) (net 43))
 (segment (start 123.25 120.275) (end 124.075001 121.100001) (width 0.25) (layer F.Cu) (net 43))
 (segment (start 123.25 118.45) (end 123.25 120.275) (width 0.25) (layer F.Cu) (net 43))
 (segment (start 123 143.75) (end 123 147) (width 0.25) (layer F.Cu) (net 44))
 (segment (start 125.10003 141.64997) (end 123 143.75) (width 0.25) (layer F.Cu) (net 44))
 (segment (start 123.25 124.575) (end 125.10003 126.42503) (width 0.25) (layer F.Cu) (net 44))
 (segment (start 125.10003 126.42503) (end 125.10003 141.64997) (width 0.25) (layer F.Cu) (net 44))
 (segment (start 123.25 123.5) (end 123.25 124.575) (width 0.25) (layer F.Cu) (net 44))
 (segment (start 121.75 143.75) (end 121.75 147) (width 0.25) (layer F.Cu) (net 45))
 (segment (start 124.65002 140.84998) (end 121.75 143.75) (width 0.25) (layer F.Cu) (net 45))
 (segment (start 122.424999 125.653589) (end 124.65002 127.87861) (width 0.25) (layer F.Cu) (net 45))
 (segment (start 124.65002 127.87861) (end 124.65002 140.84998) (width 0.25) (layer F.Cu) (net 45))
 (segment (start 122.424999 121.239999) (end 122.424999 125.653589) (width 0.25) (layer F.Cu) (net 45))
 (segment (start 120.71 119.525) (end 122.424999 121.239999) (width 0.25) (layer F.Cu) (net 45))
 (segment (start 120.71 118.45) (end 120.71 119.525) (width 0.25) (layer F.Cu) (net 45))
 (segment (start 120.5 143.75) (end 120.5 147) (width 0.25) (layer F.Cu) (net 46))
 (segment (start 124.20001 128.06501) (end 124.20001 140.04999) (width 0.25) (layer F.Cu) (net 46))
 (segment (start 120.71 124.575) (end 124.20001 128.06501) (width 0.25) (layer F.Cu) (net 46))
 (segment (start 124.20001 140.04999) (end 120.5 143.75) (width 0.25) (layer F.Cu) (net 46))
 (segment (start 120.71 123.5) (end 120.71 124.575) (width 0.25) (layer F.Cu) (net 46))
 (segment (start 119.25 143.75) (end 119.25 147) (width 0.25) (layer F.Cu) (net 47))
 (segment (start 118.17 120.275) (end 119.884999 121.989999) (width 0.25) (layer F.Cu) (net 47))
 (segment (start 118.17 118.45) (end 118.17 120.275) (width 0.25) (layer F.Cu) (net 47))
 (segment (start 119.884999 121.989999) (end 119.884999 131.134999) (width 0.25) (layer F.Cu) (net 47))
 (segment (start 119.884999 131.134999) (end 123.75 135) (width 0.25) (layer F.Cu) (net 47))
 (segment (start 123.75 135) (end 123.75 139.25) (width 0.25) (layer F.Cu) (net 47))
 (segment (start 123.75 139.25) (end 119.25 143.75) (width 0.25) (layer F.Cu) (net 47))
 (segment (start 118.17 125.325) (end 118.17 123.5) (width 0.25) (layer F.Cu) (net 48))
 (segment (start 123.25 135.13641) (end 118.17 130.05641) (width 0.25) (layer F.Cu) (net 48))
 (segment (start 118.17 130.05641) (end 118.17 125.325) (width 0.25) (layer F.Cu) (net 48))
 (segment (start 118 143.802033) (end 123.25 138.552033) (width 0.25) (layer F.Cu) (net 48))
 (segment (start 123.25 138.552033) (end 123.25 135.13641) (width 0.25) (layer F.Cu) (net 48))
 (segment (start 118 147.25) (end 118 143.802033) (width 0.25) (layer F.Cu) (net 48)))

